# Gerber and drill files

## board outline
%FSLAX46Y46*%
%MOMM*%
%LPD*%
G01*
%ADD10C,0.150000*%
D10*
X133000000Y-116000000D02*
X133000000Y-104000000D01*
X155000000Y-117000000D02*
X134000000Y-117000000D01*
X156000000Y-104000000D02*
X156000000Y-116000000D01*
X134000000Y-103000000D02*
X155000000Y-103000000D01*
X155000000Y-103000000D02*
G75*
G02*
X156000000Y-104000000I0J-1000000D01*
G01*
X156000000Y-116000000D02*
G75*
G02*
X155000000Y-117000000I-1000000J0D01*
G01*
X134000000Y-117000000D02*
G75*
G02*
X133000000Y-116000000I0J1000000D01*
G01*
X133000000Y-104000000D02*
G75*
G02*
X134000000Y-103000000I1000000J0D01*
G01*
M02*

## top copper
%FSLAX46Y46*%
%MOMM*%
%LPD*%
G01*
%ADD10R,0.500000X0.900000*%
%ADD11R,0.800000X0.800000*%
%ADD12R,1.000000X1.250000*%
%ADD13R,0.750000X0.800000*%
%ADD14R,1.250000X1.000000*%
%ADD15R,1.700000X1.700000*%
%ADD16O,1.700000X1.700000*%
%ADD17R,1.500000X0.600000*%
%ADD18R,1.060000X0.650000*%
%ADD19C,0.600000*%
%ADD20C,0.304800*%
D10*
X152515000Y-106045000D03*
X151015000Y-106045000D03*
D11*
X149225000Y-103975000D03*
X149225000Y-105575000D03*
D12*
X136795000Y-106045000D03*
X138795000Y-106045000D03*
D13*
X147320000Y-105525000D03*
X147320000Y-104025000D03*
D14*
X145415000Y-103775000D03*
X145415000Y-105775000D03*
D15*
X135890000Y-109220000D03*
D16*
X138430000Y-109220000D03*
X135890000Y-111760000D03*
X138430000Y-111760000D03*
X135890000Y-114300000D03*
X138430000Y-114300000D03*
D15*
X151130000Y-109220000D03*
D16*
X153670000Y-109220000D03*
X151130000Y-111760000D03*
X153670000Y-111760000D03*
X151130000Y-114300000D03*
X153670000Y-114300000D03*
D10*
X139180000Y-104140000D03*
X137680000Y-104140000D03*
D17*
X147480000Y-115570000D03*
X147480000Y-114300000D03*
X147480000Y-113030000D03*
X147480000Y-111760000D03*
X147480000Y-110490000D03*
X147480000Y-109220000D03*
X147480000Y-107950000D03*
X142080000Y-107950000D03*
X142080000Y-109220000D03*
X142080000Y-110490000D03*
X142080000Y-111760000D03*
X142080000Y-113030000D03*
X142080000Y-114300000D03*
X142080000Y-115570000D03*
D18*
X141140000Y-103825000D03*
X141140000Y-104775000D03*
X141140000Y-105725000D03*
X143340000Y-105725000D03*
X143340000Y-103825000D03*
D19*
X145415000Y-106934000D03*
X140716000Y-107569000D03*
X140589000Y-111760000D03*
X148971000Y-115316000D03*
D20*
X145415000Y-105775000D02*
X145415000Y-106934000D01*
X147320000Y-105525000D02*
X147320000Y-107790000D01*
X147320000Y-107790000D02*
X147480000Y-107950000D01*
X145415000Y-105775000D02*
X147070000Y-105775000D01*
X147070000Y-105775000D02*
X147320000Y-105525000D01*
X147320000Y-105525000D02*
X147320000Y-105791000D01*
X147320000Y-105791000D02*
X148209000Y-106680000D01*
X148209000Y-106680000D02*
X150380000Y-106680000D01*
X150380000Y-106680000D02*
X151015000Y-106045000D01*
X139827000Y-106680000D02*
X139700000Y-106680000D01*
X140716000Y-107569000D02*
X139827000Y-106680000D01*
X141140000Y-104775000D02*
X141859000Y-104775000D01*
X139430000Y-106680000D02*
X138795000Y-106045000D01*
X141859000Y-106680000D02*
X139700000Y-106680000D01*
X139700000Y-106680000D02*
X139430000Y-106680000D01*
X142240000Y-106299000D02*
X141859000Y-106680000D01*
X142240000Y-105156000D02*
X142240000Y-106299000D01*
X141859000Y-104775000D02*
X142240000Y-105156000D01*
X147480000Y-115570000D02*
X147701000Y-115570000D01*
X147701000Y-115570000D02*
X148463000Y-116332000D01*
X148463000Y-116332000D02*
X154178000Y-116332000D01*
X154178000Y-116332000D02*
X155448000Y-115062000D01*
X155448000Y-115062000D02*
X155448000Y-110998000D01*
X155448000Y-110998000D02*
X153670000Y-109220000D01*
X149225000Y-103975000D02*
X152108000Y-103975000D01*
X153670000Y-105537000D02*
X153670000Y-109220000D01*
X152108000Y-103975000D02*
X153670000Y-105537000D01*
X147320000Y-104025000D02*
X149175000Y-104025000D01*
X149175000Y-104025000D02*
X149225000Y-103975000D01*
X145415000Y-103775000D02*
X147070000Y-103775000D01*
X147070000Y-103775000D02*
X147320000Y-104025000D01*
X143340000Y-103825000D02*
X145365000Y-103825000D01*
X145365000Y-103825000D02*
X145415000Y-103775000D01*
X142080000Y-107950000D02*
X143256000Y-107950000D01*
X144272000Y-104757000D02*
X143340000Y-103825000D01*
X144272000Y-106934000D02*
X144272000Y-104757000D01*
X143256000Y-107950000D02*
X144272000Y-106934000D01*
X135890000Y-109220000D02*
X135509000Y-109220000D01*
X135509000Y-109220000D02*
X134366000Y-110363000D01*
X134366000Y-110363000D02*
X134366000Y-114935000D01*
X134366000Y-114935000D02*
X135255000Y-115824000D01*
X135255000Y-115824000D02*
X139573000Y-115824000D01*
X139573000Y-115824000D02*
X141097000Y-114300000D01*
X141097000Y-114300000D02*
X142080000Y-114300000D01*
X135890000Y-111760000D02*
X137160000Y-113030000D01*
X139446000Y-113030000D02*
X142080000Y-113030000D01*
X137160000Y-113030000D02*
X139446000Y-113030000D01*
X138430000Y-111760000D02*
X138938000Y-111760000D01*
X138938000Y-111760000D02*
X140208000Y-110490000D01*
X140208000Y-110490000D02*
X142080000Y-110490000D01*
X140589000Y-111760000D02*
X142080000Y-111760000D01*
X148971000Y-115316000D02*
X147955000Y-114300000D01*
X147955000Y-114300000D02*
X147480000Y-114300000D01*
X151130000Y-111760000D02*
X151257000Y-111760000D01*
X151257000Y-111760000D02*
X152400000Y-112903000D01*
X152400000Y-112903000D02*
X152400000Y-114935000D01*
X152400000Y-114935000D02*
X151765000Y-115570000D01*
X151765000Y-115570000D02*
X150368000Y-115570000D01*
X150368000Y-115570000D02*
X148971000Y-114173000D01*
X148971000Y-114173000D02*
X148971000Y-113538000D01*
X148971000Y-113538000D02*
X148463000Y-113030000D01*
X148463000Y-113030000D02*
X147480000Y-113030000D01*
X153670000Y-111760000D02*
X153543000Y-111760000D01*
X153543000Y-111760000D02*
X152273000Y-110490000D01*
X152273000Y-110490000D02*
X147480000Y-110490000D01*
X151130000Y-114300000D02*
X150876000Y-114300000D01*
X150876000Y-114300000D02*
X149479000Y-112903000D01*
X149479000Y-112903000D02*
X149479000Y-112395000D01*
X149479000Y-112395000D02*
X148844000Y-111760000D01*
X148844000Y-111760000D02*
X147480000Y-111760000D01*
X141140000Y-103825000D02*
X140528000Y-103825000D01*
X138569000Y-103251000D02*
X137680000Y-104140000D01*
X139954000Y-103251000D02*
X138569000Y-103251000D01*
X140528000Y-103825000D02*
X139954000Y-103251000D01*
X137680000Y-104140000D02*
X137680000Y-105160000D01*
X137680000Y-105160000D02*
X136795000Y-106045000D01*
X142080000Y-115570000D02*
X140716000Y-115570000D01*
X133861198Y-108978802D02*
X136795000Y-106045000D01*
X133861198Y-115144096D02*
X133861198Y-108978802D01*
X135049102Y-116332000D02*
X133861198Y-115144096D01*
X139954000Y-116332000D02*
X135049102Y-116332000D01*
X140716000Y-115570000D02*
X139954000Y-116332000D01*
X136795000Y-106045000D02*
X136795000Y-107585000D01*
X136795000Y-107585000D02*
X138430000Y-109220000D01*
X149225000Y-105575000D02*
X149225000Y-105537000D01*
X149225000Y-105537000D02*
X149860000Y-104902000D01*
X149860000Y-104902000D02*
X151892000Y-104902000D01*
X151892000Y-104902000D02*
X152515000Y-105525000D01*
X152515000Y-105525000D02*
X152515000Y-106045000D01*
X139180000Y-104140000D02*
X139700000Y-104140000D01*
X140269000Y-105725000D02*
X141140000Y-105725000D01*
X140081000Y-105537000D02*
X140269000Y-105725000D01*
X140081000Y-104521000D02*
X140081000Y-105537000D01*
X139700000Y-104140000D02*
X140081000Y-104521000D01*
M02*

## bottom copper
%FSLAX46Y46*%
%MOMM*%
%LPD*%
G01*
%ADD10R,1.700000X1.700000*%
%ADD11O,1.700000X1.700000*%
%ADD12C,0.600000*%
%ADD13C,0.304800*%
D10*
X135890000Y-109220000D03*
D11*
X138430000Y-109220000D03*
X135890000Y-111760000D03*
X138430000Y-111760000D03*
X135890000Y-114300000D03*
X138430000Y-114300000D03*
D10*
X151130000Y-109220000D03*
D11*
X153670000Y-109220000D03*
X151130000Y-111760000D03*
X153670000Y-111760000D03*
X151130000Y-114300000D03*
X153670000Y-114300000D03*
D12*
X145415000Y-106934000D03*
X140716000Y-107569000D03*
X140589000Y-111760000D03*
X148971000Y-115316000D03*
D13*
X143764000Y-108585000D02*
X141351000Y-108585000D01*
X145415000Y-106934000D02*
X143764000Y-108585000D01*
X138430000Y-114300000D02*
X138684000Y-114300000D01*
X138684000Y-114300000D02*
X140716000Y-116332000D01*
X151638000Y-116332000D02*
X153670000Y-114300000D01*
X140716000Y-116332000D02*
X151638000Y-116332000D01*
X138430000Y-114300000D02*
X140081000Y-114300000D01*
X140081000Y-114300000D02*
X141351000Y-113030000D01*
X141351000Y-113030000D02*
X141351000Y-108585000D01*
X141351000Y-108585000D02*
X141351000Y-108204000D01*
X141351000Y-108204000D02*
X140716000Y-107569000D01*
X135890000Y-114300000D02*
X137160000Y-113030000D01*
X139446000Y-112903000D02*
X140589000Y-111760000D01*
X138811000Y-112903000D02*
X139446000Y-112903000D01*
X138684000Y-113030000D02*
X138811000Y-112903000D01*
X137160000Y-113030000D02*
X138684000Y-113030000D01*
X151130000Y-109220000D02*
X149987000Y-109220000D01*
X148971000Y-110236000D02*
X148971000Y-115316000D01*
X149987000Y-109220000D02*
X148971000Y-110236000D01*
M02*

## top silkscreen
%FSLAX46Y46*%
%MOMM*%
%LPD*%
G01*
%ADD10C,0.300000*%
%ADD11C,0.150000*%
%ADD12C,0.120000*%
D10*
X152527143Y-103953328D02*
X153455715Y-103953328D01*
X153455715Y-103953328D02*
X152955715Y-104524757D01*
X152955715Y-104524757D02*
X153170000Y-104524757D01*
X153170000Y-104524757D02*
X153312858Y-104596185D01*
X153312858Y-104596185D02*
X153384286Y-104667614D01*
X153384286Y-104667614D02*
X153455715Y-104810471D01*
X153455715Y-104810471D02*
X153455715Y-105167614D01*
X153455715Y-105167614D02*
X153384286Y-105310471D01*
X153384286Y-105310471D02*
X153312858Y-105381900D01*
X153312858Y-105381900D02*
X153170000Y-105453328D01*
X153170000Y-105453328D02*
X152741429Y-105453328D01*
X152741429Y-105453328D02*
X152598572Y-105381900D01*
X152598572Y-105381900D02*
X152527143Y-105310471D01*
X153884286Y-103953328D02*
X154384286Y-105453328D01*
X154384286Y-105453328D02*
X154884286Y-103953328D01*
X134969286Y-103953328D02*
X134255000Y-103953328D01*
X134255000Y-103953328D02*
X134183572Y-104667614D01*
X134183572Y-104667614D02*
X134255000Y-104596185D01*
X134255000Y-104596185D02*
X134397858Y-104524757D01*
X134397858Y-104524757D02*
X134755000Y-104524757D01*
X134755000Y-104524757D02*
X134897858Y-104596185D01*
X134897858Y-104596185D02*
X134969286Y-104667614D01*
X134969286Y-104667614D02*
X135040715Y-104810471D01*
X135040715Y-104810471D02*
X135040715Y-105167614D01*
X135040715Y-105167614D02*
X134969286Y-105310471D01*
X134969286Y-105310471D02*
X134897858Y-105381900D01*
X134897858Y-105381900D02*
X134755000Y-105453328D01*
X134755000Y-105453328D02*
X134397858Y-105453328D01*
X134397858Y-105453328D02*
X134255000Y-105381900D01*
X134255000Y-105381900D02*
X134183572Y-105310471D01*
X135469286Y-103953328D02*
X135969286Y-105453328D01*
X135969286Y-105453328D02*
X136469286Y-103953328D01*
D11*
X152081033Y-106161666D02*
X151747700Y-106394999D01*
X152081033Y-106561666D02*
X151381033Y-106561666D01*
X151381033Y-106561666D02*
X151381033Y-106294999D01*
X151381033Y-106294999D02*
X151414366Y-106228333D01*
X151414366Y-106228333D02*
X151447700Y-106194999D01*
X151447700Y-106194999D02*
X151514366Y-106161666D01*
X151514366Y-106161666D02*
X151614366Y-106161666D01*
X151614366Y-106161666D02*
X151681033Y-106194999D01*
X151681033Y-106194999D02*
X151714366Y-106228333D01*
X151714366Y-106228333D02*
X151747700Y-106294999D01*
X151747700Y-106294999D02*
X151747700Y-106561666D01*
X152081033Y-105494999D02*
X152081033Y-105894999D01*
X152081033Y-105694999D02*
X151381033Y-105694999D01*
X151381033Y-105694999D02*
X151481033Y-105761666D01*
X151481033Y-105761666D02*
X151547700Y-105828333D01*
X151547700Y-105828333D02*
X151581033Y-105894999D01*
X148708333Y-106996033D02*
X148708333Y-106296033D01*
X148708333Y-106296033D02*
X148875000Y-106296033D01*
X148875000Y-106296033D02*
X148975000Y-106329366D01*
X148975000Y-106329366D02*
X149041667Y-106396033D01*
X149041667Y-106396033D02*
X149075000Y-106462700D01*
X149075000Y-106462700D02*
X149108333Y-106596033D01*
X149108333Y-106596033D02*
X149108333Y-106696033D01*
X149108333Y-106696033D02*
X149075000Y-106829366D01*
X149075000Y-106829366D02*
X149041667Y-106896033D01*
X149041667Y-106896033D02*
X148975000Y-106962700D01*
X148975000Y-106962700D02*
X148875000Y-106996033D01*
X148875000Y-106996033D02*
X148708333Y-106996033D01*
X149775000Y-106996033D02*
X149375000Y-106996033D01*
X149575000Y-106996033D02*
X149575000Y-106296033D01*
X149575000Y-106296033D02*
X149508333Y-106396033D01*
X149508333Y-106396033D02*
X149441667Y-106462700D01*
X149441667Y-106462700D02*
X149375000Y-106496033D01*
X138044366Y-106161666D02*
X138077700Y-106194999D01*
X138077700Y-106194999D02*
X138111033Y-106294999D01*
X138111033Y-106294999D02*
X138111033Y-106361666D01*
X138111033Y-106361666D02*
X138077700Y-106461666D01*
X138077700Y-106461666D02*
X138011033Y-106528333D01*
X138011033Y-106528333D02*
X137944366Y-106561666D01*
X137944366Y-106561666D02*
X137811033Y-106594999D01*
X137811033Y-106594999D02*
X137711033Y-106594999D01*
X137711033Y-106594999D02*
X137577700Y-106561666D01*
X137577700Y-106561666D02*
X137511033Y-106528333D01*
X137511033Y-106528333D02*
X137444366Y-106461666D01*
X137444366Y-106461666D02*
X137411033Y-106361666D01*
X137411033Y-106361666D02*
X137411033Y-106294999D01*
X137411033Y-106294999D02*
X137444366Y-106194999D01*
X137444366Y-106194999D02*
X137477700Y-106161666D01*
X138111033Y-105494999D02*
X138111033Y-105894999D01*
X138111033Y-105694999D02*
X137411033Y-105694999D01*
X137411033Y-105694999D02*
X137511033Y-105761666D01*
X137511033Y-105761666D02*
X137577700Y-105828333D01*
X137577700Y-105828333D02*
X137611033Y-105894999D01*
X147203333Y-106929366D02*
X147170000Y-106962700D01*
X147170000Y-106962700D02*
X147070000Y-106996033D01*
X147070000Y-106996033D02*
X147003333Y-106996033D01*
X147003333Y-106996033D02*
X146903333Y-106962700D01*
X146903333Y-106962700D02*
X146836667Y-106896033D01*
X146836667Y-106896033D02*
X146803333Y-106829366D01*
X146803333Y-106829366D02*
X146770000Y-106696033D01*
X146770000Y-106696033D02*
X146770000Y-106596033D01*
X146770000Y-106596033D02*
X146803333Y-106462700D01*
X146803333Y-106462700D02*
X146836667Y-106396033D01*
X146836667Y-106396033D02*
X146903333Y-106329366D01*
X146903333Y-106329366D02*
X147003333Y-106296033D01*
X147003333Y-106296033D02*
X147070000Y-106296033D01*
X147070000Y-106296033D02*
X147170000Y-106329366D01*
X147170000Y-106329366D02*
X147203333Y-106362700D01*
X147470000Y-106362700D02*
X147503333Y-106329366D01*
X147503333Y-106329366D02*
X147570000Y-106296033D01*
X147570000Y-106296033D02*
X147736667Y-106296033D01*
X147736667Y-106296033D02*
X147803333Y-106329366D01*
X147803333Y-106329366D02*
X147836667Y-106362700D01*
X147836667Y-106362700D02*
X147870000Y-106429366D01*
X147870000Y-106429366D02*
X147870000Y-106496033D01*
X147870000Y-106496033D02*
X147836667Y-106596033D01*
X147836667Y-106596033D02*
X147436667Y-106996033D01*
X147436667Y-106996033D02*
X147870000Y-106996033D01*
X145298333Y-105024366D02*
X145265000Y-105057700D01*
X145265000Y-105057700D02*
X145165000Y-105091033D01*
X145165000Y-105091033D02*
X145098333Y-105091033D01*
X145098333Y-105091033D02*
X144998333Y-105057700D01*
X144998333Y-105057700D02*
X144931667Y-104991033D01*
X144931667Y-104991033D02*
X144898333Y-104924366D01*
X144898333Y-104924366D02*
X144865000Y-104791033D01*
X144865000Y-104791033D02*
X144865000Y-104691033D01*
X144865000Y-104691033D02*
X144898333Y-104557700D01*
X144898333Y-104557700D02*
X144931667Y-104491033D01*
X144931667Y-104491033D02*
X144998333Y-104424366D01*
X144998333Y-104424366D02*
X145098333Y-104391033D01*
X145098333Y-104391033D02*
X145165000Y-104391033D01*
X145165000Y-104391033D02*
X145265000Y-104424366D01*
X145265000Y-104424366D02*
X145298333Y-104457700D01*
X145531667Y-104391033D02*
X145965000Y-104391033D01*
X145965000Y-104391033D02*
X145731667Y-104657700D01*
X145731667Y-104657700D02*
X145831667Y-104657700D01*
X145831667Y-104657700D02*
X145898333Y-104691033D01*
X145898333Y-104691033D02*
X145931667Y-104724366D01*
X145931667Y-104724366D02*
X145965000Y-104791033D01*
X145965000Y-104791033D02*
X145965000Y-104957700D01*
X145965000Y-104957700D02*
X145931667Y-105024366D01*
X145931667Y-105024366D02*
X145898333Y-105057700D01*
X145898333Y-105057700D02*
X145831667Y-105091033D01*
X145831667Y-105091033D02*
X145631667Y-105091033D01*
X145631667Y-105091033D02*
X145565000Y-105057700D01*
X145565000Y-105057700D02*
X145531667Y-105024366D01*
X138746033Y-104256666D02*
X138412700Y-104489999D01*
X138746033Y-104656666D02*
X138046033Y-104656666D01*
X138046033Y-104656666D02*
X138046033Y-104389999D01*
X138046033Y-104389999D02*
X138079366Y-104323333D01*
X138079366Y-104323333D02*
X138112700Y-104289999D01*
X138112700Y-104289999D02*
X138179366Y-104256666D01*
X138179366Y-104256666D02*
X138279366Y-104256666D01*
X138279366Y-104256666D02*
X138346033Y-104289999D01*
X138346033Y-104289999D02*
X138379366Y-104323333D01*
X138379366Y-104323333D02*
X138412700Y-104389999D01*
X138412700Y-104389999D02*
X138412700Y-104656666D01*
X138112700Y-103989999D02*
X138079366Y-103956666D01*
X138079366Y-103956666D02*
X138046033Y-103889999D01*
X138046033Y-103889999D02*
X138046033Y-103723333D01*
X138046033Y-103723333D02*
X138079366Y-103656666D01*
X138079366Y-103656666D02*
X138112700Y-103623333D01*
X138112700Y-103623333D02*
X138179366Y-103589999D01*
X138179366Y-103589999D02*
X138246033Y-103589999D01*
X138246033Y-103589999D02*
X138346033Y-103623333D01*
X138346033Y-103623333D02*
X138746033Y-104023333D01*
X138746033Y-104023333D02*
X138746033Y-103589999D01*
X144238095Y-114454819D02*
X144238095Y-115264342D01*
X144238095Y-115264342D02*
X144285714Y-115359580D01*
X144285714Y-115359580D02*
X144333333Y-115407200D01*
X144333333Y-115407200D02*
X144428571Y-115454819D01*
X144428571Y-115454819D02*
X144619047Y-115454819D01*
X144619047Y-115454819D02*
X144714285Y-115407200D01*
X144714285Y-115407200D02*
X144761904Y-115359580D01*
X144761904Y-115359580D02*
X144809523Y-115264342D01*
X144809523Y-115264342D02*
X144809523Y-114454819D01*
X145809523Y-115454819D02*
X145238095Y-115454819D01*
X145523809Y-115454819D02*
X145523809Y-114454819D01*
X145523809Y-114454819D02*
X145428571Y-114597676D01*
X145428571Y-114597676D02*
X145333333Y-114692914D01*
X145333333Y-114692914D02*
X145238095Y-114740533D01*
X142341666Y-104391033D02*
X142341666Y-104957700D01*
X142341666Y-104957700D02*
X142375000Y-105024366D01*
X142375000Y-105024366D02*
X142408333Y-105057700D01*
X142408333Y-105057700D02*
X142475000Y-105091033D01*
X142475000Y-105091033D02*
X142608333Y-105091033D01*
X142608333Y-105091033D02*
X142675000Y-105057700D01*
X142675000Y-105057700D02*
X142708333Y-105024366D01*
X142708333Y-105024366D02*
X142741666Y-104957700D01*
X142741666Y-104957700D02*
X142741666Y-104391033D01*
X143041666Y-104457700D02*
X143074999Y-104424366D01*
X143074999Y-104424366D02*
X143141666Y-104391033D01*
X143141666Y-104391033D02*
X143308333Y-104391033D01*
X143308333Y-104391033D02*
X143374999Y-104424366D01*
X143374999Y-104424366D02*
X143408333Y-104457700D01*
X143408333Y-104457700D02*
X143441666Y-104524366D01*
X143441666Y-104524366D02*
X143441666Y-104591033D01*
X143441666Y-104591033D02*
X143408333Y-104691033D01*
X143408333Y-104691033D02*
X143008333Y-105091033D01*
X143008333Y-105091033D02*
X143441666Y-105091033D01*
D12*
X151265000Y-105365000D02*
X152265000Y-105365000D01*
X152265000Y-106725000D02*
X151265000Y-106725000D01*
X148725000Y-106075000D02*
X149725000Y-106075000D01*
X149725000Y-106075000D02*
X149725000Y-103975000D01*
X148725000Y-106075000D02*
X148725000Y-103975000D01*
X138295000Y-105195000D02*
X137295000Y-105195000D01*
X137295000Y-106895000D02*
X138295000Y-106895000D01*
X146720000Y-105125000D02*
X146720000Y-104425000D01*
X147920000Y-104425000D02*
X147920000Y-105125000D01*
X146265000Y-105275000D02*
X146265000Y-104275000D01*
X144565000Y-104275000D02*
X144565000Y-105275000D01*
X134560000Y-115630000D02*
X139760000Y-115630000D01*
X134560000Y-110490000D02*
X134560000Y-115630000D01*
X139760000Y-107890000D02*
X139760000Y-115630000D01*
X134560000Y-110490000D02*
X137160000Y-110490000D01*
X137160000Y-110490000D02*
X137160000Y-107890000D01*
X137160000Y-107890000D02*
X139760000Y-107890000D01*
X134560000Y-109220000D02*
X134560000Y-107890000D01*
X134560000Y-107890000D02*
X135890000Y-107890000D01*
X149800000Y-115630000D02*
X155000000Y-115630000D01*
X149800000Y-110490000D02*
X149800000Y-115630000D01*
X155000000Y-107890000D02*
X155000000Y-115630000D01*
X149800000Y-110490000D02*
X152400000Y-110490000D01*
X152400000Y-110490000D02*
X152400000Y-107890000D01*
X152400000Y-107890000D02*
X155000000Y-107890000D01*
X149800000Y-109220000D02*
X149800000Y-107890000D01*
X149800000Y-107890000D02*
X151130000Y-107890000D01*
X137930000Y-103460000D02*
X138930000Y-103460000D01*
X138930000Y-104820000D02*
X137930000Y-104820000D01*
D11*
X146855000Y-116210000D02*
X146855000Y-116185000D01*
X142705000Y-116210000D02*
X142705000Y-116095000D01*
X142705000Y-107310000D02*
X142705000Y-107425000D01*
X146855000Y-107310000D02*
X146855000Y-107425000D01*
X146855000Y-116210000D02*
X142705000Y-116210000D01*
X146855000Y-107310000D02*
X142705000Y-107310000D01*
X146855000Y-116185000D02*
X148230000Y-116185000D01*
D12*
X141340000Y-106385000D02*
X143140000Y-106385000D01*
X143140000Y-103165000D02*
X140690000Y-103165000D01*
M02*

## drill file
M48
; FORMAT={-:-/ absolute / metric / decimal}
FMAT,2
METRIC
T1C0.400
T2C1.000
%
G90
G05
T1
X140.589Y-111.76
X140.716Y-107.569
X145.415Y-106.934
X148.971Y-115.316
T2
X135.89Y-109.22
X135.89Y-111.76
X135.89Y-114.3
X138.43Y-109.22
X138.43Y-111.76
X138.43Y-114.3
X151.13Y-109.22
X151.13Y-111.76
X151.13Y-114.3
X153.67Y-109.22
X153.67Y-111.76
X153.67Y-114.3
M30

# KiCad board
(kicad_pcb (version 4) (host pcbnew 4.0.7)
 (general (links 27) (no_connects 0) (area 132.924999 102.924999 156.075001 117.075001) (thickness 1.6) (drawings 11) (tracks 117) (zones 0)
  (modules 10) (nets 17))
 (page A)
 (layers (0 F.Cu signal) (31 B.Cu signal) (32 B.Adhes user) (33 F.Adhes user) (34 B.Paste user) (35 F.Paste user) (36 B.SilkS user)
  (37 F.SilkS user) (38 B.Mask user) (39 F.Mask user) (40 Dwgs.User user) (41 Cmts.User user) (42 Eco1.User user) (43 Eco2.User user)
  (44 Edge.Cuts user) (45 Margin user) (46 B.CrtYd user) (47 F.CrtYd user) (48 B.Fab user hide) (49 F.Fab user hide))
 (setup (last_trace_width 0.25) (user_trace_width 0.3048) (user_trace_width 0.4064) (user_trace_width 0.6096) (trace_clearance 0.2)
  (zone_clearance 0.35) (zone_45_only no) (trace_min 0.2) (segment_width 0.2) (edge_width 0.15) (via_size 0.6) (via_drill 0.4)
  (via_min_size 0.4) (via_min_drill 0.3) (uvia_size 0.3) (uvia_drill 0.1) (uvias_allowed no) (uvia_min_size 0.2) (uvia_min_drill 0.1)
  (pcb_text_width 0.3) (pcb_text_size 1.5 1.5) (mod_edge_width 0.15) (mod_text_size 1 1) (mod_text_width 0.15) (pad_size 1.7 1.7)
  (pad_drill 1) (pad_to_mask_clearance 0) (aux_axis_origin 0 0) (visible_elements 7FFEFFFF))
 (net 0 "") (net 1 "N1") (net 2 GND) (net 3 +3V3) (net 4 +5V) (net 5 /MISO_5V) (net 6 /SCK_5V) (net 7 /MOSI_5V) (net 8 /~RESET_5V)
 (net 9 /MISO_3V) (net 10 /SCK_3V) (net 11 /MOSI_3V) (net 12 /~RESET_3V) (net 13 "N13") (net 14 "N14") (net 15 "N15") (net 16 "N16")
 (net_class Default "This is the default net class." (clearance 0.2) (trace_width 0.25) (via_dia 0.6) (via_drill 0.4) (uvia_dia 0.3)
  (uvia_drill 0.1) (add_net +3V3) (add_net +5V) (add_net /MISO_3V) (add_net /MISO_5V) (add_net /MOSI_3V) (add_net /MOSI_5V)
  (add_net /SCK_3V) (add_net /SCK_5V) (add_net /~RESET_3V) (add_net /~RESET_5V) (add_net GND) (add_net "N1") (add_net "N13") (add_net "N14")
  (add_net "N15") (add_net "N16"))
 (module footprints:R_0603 (layer F.Cu) (at 151.765 106.045 180)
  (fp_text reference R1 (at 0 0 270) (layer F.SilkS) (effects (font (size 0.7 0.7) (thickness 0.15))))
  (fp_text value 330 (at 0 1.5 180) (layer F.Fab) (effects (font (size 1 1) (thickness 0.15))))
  (fp_line (start 0.5 0.68) (end -0.5 0.68) (layer F.SilkS) (width 0.12))
  (fp_line (start -0.5 -0.68) (end 0.5 -0.68) (layer F.SilkS) (width 0.12))
  (pad 1 smd rect (at -0.75 0 180) (size 0.5 0.9) (layers F.Cu F.Paste F.Mask) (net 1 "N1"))
  (pad 2 smd rect (at 0.75 0 180) (size 0.5 0.9) (layers F.Cu F.Paste F.Mask) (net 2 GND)))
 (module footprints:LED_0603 (layer F.Cu) (at 149.225 104.775 90)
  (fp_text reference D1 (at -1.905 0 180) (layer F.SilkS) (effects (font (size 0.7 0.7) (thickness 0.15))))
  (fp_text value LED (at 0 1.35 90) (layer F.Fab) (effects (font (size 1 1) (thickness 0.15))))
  (fp_line (start -1.3 -0.5) (end -1.3 0.5) (layer F.SilkS) (width 0.12))
  (fp_line (start -1.3 0.5) (end 0.8 0.5) (layer F.SilkS) (width 0.12))
  (fp_line (start -1.3 -0.5) (end 0.8 -0.5) (layer F.SilkS) (width 0.12))
  (pad 2 smd rect (at 0.8 0 270) (size 0.8 0.8) (layers F.Cu F.Paste F.Mask) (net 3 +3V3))
  (pad 1 smd rect (at -0.8 0 270) (size 0.8 0.8) (layers F.Cu F.Paste F.Mask) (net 1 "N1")))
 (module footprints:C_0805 (layer F.Cu) (at 137.795 106.045)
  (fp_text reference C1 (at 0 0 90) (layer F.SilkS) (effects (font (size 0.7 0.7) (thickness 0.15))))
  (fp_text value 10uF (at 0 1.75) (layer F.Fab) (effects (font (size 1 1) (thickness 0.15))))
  (fp_line (start 0.5 -0.85) (end -0.5 -0.85) (layer F.SilkS) (width 0.12))
  (fp_line (start -0.5 0.85) (end 0.5 0.85) (layer F.SilkS) (width 0.12))
  (pad 1 smd rect (at -1 0) (size 1 1.25) (layers F.Cu F.Paste F.Mask) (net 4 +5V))
  (pad 2 smd rect (at 1 0) (size 1 1.25) (layers F.Cu F.Paste F.Mask) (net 2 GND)))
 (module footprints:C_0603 (layer F.Cu) (at 147.32 104.775 270)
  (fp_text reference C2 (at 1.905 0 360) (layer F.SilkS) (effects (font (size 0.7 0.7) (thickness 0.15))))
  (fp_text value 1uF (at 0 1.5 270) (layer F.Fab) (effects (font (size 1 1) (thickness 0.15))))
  (fp_line (start 0.35 0.6) (end -0.35 0.6) (layer F.SilkS) (width 0.12))
  (fp_line (start -0.35 -0.6) (end 0.35 -0.6) (layer F.SilkS) (width 0.12))
  (pad 2 smd rect (at 0.75 0 270) (size 0.8 0.75) (layers F.Cu F.Paste F.Mask) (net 2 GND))
  (pad 1 smd rect (at -0.75 0 270) (size 0.8 0.75) (layers F.Cu F.Paste F.Mask) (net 3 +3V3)))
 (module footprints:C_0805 (layer F.Cu) (at 145.415 104.775 270)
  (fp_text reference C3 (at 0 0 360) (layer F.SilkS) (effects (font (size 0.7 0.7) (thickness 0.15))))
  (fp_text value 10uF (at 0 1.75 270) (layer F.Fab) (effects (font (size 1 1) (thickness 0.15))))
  (fp_line (start 0.5 -0.85) (end -0.5 -0.85) (layer F.SilkS) (width 0.12))
  (fp_line (start -0.5 0.85) (end 0.5 0.85) (layer F.SilkS) (width 0.12))
  (pad 1 smd rect (at -1 0 270) (size 1 1.25) (layers F.Cu F.Paste F.Mask) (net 3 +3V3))
  (pad 2 smd rect (at 1 0 270) (size 1 1.25) (layers F.Cu F.Paste F.Mask) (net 2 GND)))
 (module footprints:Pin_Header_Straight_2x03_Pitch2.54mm (layer F.Cu) (at 135.89 109.22)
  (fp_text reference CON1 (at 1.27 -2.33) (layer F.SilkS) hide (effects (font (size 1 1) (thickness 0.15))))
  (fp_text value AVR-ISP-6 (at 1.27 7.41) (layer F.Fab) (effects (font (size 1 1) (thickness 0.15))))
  (fp_line (start -1.33 6.41) (end 3.87 6.41) (layer F.SilkS) (width 0.12))
  (fp_line (start -1.33 1.27) (end -1.33 6.41) (layer F.SilkS) (width 0.12))
  (fp_line (start 3.87 -1.33) (end 3.87 6.41) (layer F.SilkS) (width 0.12))
  (fp_line (start -1.33 1.27) (end 1.27 1.27) (layer F.SilkS) (width 0.12))
  (fp_line (start 1.27 1.27) (end 1.27 -1.33) (layer F.SilkS) (width 0.12))
  (fp_line (start 1.27 -1.33) (end 3.87 -1.33) (layer F.SilkS) (width 0.12))
  (fp_line (start -1.33 0) (end -1.33 -1.33) (layer F.SilkS) (width 0.12))
  (fp_line (start -1.33 -1.33) (end 0 -1.33) (layer F.SilkS) (width 0.12))
  (pad 1 thru_hole rect (at 0 0) (size 1.7 1.7) (drill 1) (layers *.Cu *.Mask) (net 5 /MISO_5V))
  (pad 2 thru_hole oval (at 2.54 0) (size 1.7 1.7) (drill 1) (layers *.Cu *.Mask) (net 4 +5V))
  (pad 3 thru_hole oval (at 0 2.54) (size 1.7 1.7) (drill 1) (layers *.Cu *.Mask) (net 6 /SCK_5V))
  (pad 4 thru_hole oval (at 2.54 2.54) (size 1.7 1.7) (drill 1) (layers *.Cu *.Mask) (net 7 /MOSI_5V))
  (pad 5 thru_hole oval (at 0 5.08) (size 1.7 1.7) (drill 1) (layers *.Cu *.Mask) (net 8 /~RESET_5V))
  (pad 6 thru_hole oval (at 2.54 5.08) (size 1.7 1.7) (drill 1) (layers *.Cu *.Mask) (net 2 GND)))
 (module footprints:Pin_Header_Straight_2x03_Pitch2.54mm (layer F.Cu) (at 151.13 109.22)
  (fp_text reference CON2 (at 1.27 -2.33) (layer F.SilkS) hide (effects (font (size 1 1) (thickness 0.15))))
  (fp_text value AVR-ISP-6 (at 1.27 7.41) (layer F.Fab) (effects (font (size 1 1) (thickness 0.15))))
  (fp_line (start -1.33 6.41) (end 3.87 6.41) (layer F.SilkS) (width 0.12))
  (fp_line (start -1.33 1.27) (end -1.33 6.41) (layer F.SilkS) (width 0.12))
  (fp_line (start 3.87 -1.33) (end 3.87 6.41) (layer F.SilkS) (width 0.12))
  (fp_line (start -1.33 1.27) (end 1.27 1.27) (layer F.SilkS) (width 0.12))
  (fp_line (start 1.27 1.27) (end 1.27 -1.33) (layer F.SilkS) (width 0.12))
  (fp_line (start 1.27 -1.33) (end 3.87 -1.33) (layer F.SilkS) (width 0.12))
  (fp_line (start -1.33 0) (end -1.33 -1.33) (layer F.SilkS) (width 0.12))
  (fp_line (start -1.33 -1.33) (end 0 -1.33) (layer F.SilkS) (width 0.12))
  (pad 1 thru_hole rect (at 0 0) (size 1.7 1.7) (drill 1) (layers *.Cu *.Mask) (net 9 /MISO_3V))
  (pad 2 thru_hole oval (at 2.54 0) (size 1.7 1.7) (drill 1) (layers *.Cu *.Mask) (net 3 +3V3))
  (pad 3 thru_hole oval (at 0 2.54) (size 1.7 1.7) (drill 1) (layers *.Cu *.Mask) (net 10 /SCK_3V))
  (pad 4 thru_hole oval (at 2.54 2.54) (size 1.7 1.7) (drill 1) (layers *.Cu *.Mask) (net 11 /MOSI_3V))
  (pad 5 thru_hole oval (at 0 5.08) (size 1.7 1.7) (drill 1) (layers *.Cu *.Mask) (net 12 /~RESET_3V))
  (pad 6 thru_hole oval (at 2.54 5.08) (size 1.7 1.7) (drill 1) (layers *.Cu *.Mask) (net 2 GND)))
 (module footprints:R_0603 (layer F.Cu) (at 138.43 104.14 180)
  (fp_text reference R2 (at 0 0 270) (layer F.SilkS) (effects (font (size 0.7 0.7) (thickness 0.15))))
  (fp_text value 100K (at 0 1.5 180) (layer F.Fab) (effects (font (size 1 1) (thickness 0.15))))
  (fp_line (start 0.5 0.68) (end -0.5 0.68) (layer F.SilkS) (width 0.12))
  (fp_line (start -0.5 -0.68) (end 0.5 -0.68) (layer F.SilkS) (width 0.12))
  (pad 1 smd rect (at -0.75 0 180) (size 0.5 0.9) (layers F.Cu F.Paste F.Mask) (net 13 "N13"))
  (pad 2 smd rect (at 0.75 0 180) (size 0.5 0.9) (layers F.Cu F.Paste F.Mask) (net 4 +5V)))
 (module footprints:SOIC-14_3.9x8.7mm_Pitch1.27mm (layer F.Cu) (at 144.78 111.76 180)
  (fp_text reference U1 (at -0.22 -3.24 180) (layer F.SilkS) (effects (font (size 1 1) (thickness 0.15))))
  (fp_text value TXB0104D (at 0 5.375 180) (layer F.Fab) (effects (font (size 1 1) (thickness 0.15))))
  (fp_line (start -2.075 -4.45) (end -2.075 -4.425) (layer F.SilkS) (width 0.15))
  (fp_line (start 2.075 -4.45) (end 2.075 -4.335) (layer F.SilkS) (width 0.15))
  (fp_line (start 2.075 4.45) (end 2.075 4.335) (layer F.SilkS) (width 0.15))
  (fp_line (start -2.075 4.45) (end -2.075 4.335) (layer F.SilkS) (width 0.15))
  (fp_line (start -2.075 -4.45) (end 2.075 -4.45) (layer F.SilkS) (width 0.15))
  (fp_line (start -2.075 4.45) (end 2.075 4.45) (layer F.SilkS) (width 0.15))
  (fp_line (start -2.075 -4.425) (end -3.45 -4.425) (layer F.SilkS) (width 0.15))
  (pad 1 smd rect (at -2.7 -3.81 180) (size 1.5 0.6) (layers F.Cu F.Paste F.Mask) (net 3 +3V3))
  (pad 2 smd rect (at -2.7 -2.54 180) (size 1.5 0.6) (layers F.Cu F.Paste F.Mask) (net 9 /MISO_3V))
  (pad 3 smd rect (at -2.7 -1.27 180) (size 1.5 0.6) (layers F.Cu F.Paste F.Mask) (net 10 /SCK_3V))
  (pad 4 smd rect (at -2.7 0 180) (size 1.5 0.6) (layers F.Cu F.Paste F.Mask) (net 12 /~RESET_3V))
  (pad 5 smd rect (at -2.7 1.27 180) (size 1.5 0.6) (layers F.Cu F.Paste F.Mask) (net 11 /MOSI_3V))
  (pad 6 smd rect (at -2.7 2.54 180) (size 1.5 0.6) (layers F.Cu F.Paste F.Mask) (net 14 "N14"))
  (pad 7 smd rect (at -2.7 3.81 180) (size 1.5 0.6) (layers F.Cu F.Paste F.Mask) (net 2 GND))
  (pad 8 smd rect (at 2.7 3.81 180) (size 1.5 0.6) (layers F.Cu F.Paste F.Mask) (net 3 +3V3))
  (pad 9 smd rect (at 2.7 2.54 180) (size 1.5 0.6) (layers F.Cu F.Paste F.Mask) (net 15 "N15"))
  (pad 10 smd rect (at 2.7 1.27 180) (size 1.5 0.6) (layers F.Cu F.Paste F.Mask) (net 7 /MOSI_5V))
  (pad 11 smd rect (at 2.7 0 180) (size 1.5 0.6) (layers F.Cu F.Paste F.Mask) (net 8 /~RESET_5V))
  (pad 12 smd rect (at 2.7 -1.27 180) (size 1.5 0.6) (layers F.Cu F.Paste F.Mask) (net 6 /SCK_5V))
  (pad 13 smd rect (at 2.7 -2.54 180) (size 1.5 0.6) (layers F.Cu F.Paste F.Mask) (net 5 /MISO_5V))
  (pad 14 smd rect (at 2.7 -3.81 180) (size 1.5 0.6) (layers F.Cu F.Paste F.Mask) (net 4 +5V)))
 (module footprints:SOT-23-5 (layer F.Cu) (at 142.24 104.775)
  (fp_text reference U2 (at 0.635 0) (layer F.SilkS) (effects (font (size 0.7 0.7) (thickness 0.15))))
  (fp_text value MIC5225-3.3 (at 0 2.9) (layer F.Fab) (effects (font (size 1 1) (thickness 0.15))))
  (fp_line (start -0.9 1.61) (end 0.9 1.61) (layer F.SilkS) (width 0.12))
  (fp_line (start 0.9 -1.61) (end -1.55 -1.61) (layer F.SilkS) (width 0.12))
  (pad 1 smd rect (at -1.1 -0.95) (size 1.06 0.65) (layers F.Cu F.Paste F.Mask) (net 4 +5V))
  (pad 2 smd rect (at -1.1 0) (size 1.06 0.65) (layers F.Cu F.Paste F.Mask) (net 2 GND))
  (pad 3 smd rect (at -1.1 0.95) (size 1.06 0.65) (layers F.Cu F.Paste F.Mask) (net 13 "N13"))
  (pad 4 smd rect (at 1.1 0.95) (size 1.06 0.65) (layers F.Cu F.Paste F.Mask) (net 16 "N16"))
  (pad 5 smd rect (at 1.1 -0.95) (size 1.06 0.65) (layers F.Cu F.Paste F.Mask) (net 3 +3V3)))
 (gr_line (start 133 116) (end 133 104) (angle 90) (layer Edge.Cuts) (width 0.15))
 (gr_line (start 155 117) (end 134 117) (angle 90) (layer Edge.Cuts) (width 0.15))
 (gr_line (start 156 104) (end 156 116) (angle 90) (layer Edge.Cuts) (width 0.15))
 (gr_line (start 134 103) (end 155 103) (angle 90) (layer Edge.Cuts) (width 0.15))
 (gr_arc (start 155 104) (end 155 103) (angle 90) (layer Edge.Cuts) (width 0.15))
 (gr_arc (start 155 116) (end 156 116) (angle 90) (layer Edge.Cuts) (width 0.15))
 (gr_arc (start 134 116) (end 134 117) (angle 90) (layer Edge.Cuts) (width 0.15))
 (gr_arc (start 134 104) (end 133 104) (angle 90) (layer Edge.Cuts) (width 0.15))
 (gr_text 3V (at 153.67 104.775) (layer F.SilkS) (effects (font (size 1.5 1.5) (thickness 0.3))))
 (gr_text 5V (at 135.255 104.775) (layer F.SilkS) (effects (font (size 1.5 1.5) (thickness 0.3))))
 (segment (start 145.415 105.775) (end 145.415 106.934) (width 0.3048) (layer F.Cu) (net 2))
 (segment (start 143.764 108.585) (end 141.351 108.585) (width 0.3048) (layer B.Cu) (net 2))
 (segment (start 145.415 106.934) (end 143.764 108.585) (width 0.3048) (layer B.Cu) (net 2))
 (via (at 145.415 106.934) (size 0.6) (drill 0.4) (layers F.Cu B.Cu) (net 2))
 (segment (start 147.32 105.525) (end 147.32 107.79) (width 0.3048) (layer F.Cu) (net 2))
 (segment (start 147.32 107.79) (end 147.48 107.95) (width 0.3048) (layer F.Cu) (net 2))
 (segment (start 145.415 105.775) (end 147.07 105.775) (width 0.3048) (layer F.Cu) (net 2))
 (segment (start 147.07 105.775) (end 147.32 105.525) (width 0.3048) (layer F.Cu) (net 2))
 (segment (start 138.43 114.3) (end 138.684 114.3) (width 0.3048) (layer B.Cu) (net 2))
 (segment (start 138.684 114.3) (end 140.716 116.332) (width 0.3048) (layer B.Cu) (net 2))
 (segment (start 151.638 116.332) (end 153.67 114.3) (width 0.3048) (layer B.Cu) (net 2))
 (segment (start 140.716 116.332) (end 151.638 116.332) (width 0.3048) (layer B.Cu) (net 2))
 (segment (start 147.32 105.525) (end 147.32 105.791) (width 0.3048) (layer F.Cu) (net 2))
 (segment (start 147.32 105.791) (end 148.209 106.68) (width 0.3048) (layer F.Cu) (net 2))
 (segment (start 148.209 106.68) (end 150.38 106.68) (width 0.3048) (layer F.Cu) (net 2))
 (segment (start 150.38 106.68) (end 151.015 106.045) (width 0.3048) (layer F.Cu) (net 2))
 (segment (start 138.43 114.3) (end 140.081 114.3) (width 0.3048) (layer B.Cu) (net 2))
 (segment (start 140.081 114.3) (end 141.351 113.03) (width 0.3048) (layer B.Cu) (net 2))
 (segment (start 141.351 113.03) (end 141.351 108.585) (width 0.3048) (layer B.Cu) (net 2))
 (segment (start 139.827 106.68) (end 139.7 106.68) (width 0.3048) (layer F.Cu) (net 2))
 (segment (start 141.351 108.585) (end 141.351 108.204) (width 0.3048) (layer B.Cu) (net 2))
 (segment (start 141.351 108.204) (end 140.716 107.569) (width 0.3048) (layer B.Cu) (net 2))
 (via (at 140.716 107.569) (size 0.6) (drill 0.4) (layers F.Cu B.Cu) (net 2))
 (segment (start 140.716 107.569) (end 139.827 106.68) (width 0.3048) (layer F.Cu) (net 2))
 (segment (start 141.14 104.775) (end 141.859 104.775) (width 0.3048) (layer F.Cu) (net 2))
 (segment (start 139.43 106.68) (end 138.795 106.045) (width 0.3048) (layer F.Cu) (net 2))
 (segment (start 141.859 106.68) (end 139.7 106.68) (width 0.3048) (layer F.Cu) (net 2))
 (segment (start 139.7 106.68) (end 139.43 106.68) (width 0.3048) (layer F.Cu) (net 2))
 (segment (start 142.24 106.299) (end 141.859 106.68) (width 0.3048) (layer F.Cu) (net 2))
 (segment (start 142.24 105.156) (end 142.24 106.299) (width 0.3048) (layer F.Cu) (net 2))
 (segment (start 141.859 104.775) (end 142.24 105.156) (width 0.3048) (layer F.Cu) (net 2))
 (segment (start 147.48 115.57) (end 147.701 115.57) (width 0.3048) (layer F.Cu) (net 3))
 (segment (start 147.701 115.57) (end 148.463 116.332) (width 0.3048) (layer F.Cu) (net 3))
 (segment (start 148.463 116.332) (end 154.178 116.332) (width 0.3048) (layer F.Cu) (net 3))
 (segment (start 154.178 116.332) (end 155.448 115.062) (width 0.3048) (layer F.Cu) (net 3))
 (segment (start 155.448 115.062) (end 155.448 110.998) (width 0.3048) (layer F.Cu) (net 3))
 (segment (start 155.448 110.998) (end 153.67 109.22) (width 0.3048) (layer F.Cu) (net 3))
 (segment (start 149.225 103.975) (end 152.108 103.975) (width 0.3048) (layer F.Cu) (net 3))
 (segment (start 153.67 105.537) (end 153.67 109.22) (width 0.3048) (layer F.Cu) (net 3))
 (segment (start 152.108 103.975) (end 153.67 105.537) (width 0.3048) (layer F.Cu) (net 3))
 (segment (start 147.32 104.025) (end 149.175 104.025) (width 0.3048) (layer F.Cu) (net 3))
 (segment (start 149.175 104.025) (end 149.225 103.975) (width 0.3048) (layer F.Cu) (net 3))
 (segment (start 145.415 103.775) (end 147.07 103.775) (width 0.3048) (layer F.Cu) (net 3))
 (segment (start 147.07 103.775) (end 147.32 104.025) (width 0.3048) (layer F.Cu) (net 3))
 (segment (start 143.34 103.825) (end 145.365 103.825) (width 0.3048) (layer F.Cu) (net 3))
 (segment (start 145.365 103.825) (end 145.415 103.775) (width 0.3048) (layer F.Cu) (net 3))
 (segment (start 142.08 107.95) (end 143.256 107.95) (width 0.3048) (layer F.Cu) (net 3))
 (segment (start 144.272 104.757) (end 143.34 103.825) (width 0.3048) (layer F.Cu) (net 3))
 (segment (start 144.272 106.934) (end 144.272 104.757) (width 0.3048) (layer F.Cu) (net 3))
 (segment (start 143.256 107.95) (end 144.272 106.934) (width 0.3048) (layer F.Cu) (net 3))
 (segment (start 135.89 109.22) (end 135.509 109.22) (width 0.3048) (layer F.Cu) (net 5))
 (segment (start 135.509 109.22) (end 134.366 110.363) (width 0.3048) (layer F.Cu) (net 5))
 (segment (start 134.366 110.363) (end 134.366 114.935) (width 0.3048) (layer F.Cu) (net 5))
 (segment (start 134.366 114.935) (end 135.255 115.824) (width 0.3048) (layer F.Cu) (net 5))
 (segment (start 135.255 115.824) (end 139.573 115.824) (width 0.3048) (layer F.Cu) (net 5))
 (segment (start 139.573 115.824) (end 141.097 114.3) (width 0.3048) (layer F.Cu) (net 5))
 (segment (start 141.097 114.3) (end 142.08 114.3) (width 0.3048) (layer F.Cu) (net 5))
 (segment (start 135.89 111.76) (end 137.16 113.03) (width 0.3048) (layer F.Cu) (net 6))
 (segment (start 139.446 113.03) (end 142.08 113.03) (width 0.3048) (layer F.Cu) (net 6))
 (segment (start 137.16 113.03) (end 139.446 113.03) (width 0.3048) (layer F.Cu) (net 6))
 (segment (start 138.43 111.76) (end 138.938 111.76) (width 0.3048) (layer F.Cu) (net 7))
 (segment (start 138.938 111.76) (end 140.208 110.49) (width 0.3048) (layer F.Cu) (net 7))
 (segment (start 140.208 110.49) (end 142.08 110.49) (width 0.3048) (layer F.Cu) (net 7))
 (segment (start 135.89 114.3) (end 137.16 113.03) (width 0.3048) (layer B.Cu) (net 8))
 (segment (start 140.589 111.76) (end 142.08 111.76) (width 0.3048) (layer F.Cu) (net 8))
 (via (at 140.589 111.76) (size 0.6) (drill 0.4) (layers F.Cu B.Cu) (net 8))
 (segment (start 139.446 112.903) (end 140.589 111.76) (width 0.3048) (layer B.Cu) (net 8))
 (segment (start 138.811 112.903) (end 139.446 112.903) (width 0.3048) (layer B.Cu) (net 8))
 (segment (start 138.684 113.03) (end 138.811 112.903) (width 0.3048) (layer B.Cu) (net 8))
 (segment (start 137.16 113.03) (end 138.684 113.03) (width 0.3048) (layer B.Cu) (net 8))
 (segment (start 151.13 109.22) (end 149.987 109.22) (width 0.3048) (layer B.Cu) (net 9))
 (segment (start 148.971 115.316) (end 147.955 114.3) (width 0.3048) (layer F.Cu) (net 9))
 (via (at 148.971 115.316) (size 0.6) (drill 0.4) (layers F.Cu B.Cu) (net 9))
 (segment (start 148.971 110.236) (end 148.971 115.316) (width 0.3048) (layer B.Cu) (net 9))
 (segment (start 149.987 109.22) (end 148.971 110.236) (width 0.3048) (layer B.Cu) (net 9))
 (segment (start 147.955 114.3) (end 147.48 114.3) (width 0.3048) (layer F.Cu) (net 9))
 (segment (start 151.13 111.76) (end 151.257 111.76) (width 0.3048) (layer F.Cu) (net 10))
 (segment (start 151.257 111.76) (end 152.4 112.903) (width 0.3048) (layer F.Cu) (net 10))
 (segment (start 152.4 112.903) (end 152.4 114.935) (width 0.3048) (layer F.Cu) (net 10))
 (segment (start 152.4 114.935) (end 151.765 115.57) (width 0.3048) (layer F.Cu) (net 10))
 (segment (start 151.765 115.57) (end 150.368 115.57) (width 0.3048) (layer F.Cu) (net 10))
 (segment (start 150.368 115.57) (end 148.971 114.173) (width 0.3048) (layer F.Cu) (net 10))
 (segment (start 148.971 114.173) (end 148.971 113.538) (width 0.3048) (layer F.Cu) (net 10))
 (segment (start 148.971 113.538) (end 148.463 113.03) (width 0.3048) (layer F.Cu) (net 10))
 (segment (start 148.463 113.03) (end 147.48 113.03) (width 0.3048) (layer F.Cu) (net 10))
 (segment (start 153.67 111.76) (end 153.543 111.76) (width 0.3048) (layer F.Cu) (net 11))
 (segment (start 153.543 111.76) (end 152.273 110.49) (width 0.3048) (layer F.Cu) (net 11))
 (segment (start 152.273 110.49) (end 147.48 110.49) (width 0.3048) (layer F.Cu) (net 11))
 (segment (start 151.13 114.3) (end 150.876 114.3) (width 0.3048) (layer F.Cu) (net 12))
 (segment (start 150.876 114.3) (end 149.479 112.903) (width 0.3048) (layer F.Cu) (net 12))
 (segment (start 149.479 112.903) (end 149.479 112.395) (width 0.3048) (layer F.Cu) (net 12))
 (segment (start 149.479 112.395) (end 148.844 111.76) (width 0.3048) (layer F.Cu) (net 12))
 (segment (start 148.844 111.76) (end 147.48 111.76) (width 0.3048) (layer F.Cu) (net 12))
 (segment (start 141.14 103.825) (end 140.528 103.825) (width 0.3048) (layer F.Cu) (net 4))
 (segment (start 138.569 103.251) (end 137.68 104.14) (width 0.3048) (layer F.Cu) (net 4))
 (segment (start 139.954 103.251) (end 138.569 103.251) (width 0.3048) (layer F.Cu) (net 4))
 (segment (start 140.528 103.825) (end 139.954 103.251) (width 0.3048) (layer F.Cu) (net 4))
 (segment (start 137.68 104.14) (end 137.68 105.16) (width 0.3048) (layer F.Cu) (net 4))
 (segment (start 137.68 105.16) (end 136.795 106.045) (width 0.3048) (layer F.Cu) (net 4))
 (segment (start 142.08 115.57) (end 140.716 115.57) (width 0.3048) (layer F.Cu) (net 4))
 (segment (start 133.861198 108.978802) (end 136.795 106.045) (width 0.3048) (layer F.Cu) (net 4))
 (segment (start 133.861198 115.144096) (end 133.861198 108.978802) (width 0.3048) (layer F.Cu) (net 4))
 (segment (start 135.049102 116.332) (end 133.861198 115.144096) (width 0.3048) (layer F.Cu) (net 4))
 (segment (start 139.954 116.332) (end 135.049102 116.332) (width 0.3048) (layer F.Cu) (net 4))
 (segment (start 140.716 115.57) (end 139.954 116.332) (width 0.3048) (layer F.Cu) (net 4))
 (segment (start 136.795 106.045) (end 136.795 107.585) (width 0.3048) (layer F.Cu) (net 4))
 (segment (start 136.795 107.585) (end 138.43 109.22) (width 0.3048) (layer F.Cu) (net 4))
 (segment (start 149.225 105.575) (end 149.225 105.537) (width 0.3048) (layer F.Cu) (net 1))
 (segment (start 149.225 105.537) (end 149.86 104.902) (width 0.3048) (layer F.Cu) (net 1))
 (segment (start 149.86 104.902) (end 151.892 104.902) (width 0.3048) (layer F.Cu) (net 1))
 (segment (start 151.892 104.902) (end 152.515 105.525) (width 0.3048) (layer F.Cu) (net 1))
 (segment (start 152.515 105.525) (end 152.515 106.045) (width 0.3048) (layer F.Cu) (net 1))
 (segment (start 139.18 104.14) (end 139.7 104.14) (width 0.3048) (layer F.Cu) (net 13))
 (segment (start 140.269 105.725) (end 141.14 105.725) (width 0.3048) (layer F.Cu) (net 13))
 (segment (start 140.081 105.537) (end 140.269 105.725) (width 0.3048) (layer F.Cu) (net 13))
 (segment (start 140.081 104.521) (end 140.081 105.537) (width 0.3048) (layer F.Cu) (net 13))
 (segment (start 139.7 104.14) (end 140.081 104.521) (width 0.3048) (layer F.Cu) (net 13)))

